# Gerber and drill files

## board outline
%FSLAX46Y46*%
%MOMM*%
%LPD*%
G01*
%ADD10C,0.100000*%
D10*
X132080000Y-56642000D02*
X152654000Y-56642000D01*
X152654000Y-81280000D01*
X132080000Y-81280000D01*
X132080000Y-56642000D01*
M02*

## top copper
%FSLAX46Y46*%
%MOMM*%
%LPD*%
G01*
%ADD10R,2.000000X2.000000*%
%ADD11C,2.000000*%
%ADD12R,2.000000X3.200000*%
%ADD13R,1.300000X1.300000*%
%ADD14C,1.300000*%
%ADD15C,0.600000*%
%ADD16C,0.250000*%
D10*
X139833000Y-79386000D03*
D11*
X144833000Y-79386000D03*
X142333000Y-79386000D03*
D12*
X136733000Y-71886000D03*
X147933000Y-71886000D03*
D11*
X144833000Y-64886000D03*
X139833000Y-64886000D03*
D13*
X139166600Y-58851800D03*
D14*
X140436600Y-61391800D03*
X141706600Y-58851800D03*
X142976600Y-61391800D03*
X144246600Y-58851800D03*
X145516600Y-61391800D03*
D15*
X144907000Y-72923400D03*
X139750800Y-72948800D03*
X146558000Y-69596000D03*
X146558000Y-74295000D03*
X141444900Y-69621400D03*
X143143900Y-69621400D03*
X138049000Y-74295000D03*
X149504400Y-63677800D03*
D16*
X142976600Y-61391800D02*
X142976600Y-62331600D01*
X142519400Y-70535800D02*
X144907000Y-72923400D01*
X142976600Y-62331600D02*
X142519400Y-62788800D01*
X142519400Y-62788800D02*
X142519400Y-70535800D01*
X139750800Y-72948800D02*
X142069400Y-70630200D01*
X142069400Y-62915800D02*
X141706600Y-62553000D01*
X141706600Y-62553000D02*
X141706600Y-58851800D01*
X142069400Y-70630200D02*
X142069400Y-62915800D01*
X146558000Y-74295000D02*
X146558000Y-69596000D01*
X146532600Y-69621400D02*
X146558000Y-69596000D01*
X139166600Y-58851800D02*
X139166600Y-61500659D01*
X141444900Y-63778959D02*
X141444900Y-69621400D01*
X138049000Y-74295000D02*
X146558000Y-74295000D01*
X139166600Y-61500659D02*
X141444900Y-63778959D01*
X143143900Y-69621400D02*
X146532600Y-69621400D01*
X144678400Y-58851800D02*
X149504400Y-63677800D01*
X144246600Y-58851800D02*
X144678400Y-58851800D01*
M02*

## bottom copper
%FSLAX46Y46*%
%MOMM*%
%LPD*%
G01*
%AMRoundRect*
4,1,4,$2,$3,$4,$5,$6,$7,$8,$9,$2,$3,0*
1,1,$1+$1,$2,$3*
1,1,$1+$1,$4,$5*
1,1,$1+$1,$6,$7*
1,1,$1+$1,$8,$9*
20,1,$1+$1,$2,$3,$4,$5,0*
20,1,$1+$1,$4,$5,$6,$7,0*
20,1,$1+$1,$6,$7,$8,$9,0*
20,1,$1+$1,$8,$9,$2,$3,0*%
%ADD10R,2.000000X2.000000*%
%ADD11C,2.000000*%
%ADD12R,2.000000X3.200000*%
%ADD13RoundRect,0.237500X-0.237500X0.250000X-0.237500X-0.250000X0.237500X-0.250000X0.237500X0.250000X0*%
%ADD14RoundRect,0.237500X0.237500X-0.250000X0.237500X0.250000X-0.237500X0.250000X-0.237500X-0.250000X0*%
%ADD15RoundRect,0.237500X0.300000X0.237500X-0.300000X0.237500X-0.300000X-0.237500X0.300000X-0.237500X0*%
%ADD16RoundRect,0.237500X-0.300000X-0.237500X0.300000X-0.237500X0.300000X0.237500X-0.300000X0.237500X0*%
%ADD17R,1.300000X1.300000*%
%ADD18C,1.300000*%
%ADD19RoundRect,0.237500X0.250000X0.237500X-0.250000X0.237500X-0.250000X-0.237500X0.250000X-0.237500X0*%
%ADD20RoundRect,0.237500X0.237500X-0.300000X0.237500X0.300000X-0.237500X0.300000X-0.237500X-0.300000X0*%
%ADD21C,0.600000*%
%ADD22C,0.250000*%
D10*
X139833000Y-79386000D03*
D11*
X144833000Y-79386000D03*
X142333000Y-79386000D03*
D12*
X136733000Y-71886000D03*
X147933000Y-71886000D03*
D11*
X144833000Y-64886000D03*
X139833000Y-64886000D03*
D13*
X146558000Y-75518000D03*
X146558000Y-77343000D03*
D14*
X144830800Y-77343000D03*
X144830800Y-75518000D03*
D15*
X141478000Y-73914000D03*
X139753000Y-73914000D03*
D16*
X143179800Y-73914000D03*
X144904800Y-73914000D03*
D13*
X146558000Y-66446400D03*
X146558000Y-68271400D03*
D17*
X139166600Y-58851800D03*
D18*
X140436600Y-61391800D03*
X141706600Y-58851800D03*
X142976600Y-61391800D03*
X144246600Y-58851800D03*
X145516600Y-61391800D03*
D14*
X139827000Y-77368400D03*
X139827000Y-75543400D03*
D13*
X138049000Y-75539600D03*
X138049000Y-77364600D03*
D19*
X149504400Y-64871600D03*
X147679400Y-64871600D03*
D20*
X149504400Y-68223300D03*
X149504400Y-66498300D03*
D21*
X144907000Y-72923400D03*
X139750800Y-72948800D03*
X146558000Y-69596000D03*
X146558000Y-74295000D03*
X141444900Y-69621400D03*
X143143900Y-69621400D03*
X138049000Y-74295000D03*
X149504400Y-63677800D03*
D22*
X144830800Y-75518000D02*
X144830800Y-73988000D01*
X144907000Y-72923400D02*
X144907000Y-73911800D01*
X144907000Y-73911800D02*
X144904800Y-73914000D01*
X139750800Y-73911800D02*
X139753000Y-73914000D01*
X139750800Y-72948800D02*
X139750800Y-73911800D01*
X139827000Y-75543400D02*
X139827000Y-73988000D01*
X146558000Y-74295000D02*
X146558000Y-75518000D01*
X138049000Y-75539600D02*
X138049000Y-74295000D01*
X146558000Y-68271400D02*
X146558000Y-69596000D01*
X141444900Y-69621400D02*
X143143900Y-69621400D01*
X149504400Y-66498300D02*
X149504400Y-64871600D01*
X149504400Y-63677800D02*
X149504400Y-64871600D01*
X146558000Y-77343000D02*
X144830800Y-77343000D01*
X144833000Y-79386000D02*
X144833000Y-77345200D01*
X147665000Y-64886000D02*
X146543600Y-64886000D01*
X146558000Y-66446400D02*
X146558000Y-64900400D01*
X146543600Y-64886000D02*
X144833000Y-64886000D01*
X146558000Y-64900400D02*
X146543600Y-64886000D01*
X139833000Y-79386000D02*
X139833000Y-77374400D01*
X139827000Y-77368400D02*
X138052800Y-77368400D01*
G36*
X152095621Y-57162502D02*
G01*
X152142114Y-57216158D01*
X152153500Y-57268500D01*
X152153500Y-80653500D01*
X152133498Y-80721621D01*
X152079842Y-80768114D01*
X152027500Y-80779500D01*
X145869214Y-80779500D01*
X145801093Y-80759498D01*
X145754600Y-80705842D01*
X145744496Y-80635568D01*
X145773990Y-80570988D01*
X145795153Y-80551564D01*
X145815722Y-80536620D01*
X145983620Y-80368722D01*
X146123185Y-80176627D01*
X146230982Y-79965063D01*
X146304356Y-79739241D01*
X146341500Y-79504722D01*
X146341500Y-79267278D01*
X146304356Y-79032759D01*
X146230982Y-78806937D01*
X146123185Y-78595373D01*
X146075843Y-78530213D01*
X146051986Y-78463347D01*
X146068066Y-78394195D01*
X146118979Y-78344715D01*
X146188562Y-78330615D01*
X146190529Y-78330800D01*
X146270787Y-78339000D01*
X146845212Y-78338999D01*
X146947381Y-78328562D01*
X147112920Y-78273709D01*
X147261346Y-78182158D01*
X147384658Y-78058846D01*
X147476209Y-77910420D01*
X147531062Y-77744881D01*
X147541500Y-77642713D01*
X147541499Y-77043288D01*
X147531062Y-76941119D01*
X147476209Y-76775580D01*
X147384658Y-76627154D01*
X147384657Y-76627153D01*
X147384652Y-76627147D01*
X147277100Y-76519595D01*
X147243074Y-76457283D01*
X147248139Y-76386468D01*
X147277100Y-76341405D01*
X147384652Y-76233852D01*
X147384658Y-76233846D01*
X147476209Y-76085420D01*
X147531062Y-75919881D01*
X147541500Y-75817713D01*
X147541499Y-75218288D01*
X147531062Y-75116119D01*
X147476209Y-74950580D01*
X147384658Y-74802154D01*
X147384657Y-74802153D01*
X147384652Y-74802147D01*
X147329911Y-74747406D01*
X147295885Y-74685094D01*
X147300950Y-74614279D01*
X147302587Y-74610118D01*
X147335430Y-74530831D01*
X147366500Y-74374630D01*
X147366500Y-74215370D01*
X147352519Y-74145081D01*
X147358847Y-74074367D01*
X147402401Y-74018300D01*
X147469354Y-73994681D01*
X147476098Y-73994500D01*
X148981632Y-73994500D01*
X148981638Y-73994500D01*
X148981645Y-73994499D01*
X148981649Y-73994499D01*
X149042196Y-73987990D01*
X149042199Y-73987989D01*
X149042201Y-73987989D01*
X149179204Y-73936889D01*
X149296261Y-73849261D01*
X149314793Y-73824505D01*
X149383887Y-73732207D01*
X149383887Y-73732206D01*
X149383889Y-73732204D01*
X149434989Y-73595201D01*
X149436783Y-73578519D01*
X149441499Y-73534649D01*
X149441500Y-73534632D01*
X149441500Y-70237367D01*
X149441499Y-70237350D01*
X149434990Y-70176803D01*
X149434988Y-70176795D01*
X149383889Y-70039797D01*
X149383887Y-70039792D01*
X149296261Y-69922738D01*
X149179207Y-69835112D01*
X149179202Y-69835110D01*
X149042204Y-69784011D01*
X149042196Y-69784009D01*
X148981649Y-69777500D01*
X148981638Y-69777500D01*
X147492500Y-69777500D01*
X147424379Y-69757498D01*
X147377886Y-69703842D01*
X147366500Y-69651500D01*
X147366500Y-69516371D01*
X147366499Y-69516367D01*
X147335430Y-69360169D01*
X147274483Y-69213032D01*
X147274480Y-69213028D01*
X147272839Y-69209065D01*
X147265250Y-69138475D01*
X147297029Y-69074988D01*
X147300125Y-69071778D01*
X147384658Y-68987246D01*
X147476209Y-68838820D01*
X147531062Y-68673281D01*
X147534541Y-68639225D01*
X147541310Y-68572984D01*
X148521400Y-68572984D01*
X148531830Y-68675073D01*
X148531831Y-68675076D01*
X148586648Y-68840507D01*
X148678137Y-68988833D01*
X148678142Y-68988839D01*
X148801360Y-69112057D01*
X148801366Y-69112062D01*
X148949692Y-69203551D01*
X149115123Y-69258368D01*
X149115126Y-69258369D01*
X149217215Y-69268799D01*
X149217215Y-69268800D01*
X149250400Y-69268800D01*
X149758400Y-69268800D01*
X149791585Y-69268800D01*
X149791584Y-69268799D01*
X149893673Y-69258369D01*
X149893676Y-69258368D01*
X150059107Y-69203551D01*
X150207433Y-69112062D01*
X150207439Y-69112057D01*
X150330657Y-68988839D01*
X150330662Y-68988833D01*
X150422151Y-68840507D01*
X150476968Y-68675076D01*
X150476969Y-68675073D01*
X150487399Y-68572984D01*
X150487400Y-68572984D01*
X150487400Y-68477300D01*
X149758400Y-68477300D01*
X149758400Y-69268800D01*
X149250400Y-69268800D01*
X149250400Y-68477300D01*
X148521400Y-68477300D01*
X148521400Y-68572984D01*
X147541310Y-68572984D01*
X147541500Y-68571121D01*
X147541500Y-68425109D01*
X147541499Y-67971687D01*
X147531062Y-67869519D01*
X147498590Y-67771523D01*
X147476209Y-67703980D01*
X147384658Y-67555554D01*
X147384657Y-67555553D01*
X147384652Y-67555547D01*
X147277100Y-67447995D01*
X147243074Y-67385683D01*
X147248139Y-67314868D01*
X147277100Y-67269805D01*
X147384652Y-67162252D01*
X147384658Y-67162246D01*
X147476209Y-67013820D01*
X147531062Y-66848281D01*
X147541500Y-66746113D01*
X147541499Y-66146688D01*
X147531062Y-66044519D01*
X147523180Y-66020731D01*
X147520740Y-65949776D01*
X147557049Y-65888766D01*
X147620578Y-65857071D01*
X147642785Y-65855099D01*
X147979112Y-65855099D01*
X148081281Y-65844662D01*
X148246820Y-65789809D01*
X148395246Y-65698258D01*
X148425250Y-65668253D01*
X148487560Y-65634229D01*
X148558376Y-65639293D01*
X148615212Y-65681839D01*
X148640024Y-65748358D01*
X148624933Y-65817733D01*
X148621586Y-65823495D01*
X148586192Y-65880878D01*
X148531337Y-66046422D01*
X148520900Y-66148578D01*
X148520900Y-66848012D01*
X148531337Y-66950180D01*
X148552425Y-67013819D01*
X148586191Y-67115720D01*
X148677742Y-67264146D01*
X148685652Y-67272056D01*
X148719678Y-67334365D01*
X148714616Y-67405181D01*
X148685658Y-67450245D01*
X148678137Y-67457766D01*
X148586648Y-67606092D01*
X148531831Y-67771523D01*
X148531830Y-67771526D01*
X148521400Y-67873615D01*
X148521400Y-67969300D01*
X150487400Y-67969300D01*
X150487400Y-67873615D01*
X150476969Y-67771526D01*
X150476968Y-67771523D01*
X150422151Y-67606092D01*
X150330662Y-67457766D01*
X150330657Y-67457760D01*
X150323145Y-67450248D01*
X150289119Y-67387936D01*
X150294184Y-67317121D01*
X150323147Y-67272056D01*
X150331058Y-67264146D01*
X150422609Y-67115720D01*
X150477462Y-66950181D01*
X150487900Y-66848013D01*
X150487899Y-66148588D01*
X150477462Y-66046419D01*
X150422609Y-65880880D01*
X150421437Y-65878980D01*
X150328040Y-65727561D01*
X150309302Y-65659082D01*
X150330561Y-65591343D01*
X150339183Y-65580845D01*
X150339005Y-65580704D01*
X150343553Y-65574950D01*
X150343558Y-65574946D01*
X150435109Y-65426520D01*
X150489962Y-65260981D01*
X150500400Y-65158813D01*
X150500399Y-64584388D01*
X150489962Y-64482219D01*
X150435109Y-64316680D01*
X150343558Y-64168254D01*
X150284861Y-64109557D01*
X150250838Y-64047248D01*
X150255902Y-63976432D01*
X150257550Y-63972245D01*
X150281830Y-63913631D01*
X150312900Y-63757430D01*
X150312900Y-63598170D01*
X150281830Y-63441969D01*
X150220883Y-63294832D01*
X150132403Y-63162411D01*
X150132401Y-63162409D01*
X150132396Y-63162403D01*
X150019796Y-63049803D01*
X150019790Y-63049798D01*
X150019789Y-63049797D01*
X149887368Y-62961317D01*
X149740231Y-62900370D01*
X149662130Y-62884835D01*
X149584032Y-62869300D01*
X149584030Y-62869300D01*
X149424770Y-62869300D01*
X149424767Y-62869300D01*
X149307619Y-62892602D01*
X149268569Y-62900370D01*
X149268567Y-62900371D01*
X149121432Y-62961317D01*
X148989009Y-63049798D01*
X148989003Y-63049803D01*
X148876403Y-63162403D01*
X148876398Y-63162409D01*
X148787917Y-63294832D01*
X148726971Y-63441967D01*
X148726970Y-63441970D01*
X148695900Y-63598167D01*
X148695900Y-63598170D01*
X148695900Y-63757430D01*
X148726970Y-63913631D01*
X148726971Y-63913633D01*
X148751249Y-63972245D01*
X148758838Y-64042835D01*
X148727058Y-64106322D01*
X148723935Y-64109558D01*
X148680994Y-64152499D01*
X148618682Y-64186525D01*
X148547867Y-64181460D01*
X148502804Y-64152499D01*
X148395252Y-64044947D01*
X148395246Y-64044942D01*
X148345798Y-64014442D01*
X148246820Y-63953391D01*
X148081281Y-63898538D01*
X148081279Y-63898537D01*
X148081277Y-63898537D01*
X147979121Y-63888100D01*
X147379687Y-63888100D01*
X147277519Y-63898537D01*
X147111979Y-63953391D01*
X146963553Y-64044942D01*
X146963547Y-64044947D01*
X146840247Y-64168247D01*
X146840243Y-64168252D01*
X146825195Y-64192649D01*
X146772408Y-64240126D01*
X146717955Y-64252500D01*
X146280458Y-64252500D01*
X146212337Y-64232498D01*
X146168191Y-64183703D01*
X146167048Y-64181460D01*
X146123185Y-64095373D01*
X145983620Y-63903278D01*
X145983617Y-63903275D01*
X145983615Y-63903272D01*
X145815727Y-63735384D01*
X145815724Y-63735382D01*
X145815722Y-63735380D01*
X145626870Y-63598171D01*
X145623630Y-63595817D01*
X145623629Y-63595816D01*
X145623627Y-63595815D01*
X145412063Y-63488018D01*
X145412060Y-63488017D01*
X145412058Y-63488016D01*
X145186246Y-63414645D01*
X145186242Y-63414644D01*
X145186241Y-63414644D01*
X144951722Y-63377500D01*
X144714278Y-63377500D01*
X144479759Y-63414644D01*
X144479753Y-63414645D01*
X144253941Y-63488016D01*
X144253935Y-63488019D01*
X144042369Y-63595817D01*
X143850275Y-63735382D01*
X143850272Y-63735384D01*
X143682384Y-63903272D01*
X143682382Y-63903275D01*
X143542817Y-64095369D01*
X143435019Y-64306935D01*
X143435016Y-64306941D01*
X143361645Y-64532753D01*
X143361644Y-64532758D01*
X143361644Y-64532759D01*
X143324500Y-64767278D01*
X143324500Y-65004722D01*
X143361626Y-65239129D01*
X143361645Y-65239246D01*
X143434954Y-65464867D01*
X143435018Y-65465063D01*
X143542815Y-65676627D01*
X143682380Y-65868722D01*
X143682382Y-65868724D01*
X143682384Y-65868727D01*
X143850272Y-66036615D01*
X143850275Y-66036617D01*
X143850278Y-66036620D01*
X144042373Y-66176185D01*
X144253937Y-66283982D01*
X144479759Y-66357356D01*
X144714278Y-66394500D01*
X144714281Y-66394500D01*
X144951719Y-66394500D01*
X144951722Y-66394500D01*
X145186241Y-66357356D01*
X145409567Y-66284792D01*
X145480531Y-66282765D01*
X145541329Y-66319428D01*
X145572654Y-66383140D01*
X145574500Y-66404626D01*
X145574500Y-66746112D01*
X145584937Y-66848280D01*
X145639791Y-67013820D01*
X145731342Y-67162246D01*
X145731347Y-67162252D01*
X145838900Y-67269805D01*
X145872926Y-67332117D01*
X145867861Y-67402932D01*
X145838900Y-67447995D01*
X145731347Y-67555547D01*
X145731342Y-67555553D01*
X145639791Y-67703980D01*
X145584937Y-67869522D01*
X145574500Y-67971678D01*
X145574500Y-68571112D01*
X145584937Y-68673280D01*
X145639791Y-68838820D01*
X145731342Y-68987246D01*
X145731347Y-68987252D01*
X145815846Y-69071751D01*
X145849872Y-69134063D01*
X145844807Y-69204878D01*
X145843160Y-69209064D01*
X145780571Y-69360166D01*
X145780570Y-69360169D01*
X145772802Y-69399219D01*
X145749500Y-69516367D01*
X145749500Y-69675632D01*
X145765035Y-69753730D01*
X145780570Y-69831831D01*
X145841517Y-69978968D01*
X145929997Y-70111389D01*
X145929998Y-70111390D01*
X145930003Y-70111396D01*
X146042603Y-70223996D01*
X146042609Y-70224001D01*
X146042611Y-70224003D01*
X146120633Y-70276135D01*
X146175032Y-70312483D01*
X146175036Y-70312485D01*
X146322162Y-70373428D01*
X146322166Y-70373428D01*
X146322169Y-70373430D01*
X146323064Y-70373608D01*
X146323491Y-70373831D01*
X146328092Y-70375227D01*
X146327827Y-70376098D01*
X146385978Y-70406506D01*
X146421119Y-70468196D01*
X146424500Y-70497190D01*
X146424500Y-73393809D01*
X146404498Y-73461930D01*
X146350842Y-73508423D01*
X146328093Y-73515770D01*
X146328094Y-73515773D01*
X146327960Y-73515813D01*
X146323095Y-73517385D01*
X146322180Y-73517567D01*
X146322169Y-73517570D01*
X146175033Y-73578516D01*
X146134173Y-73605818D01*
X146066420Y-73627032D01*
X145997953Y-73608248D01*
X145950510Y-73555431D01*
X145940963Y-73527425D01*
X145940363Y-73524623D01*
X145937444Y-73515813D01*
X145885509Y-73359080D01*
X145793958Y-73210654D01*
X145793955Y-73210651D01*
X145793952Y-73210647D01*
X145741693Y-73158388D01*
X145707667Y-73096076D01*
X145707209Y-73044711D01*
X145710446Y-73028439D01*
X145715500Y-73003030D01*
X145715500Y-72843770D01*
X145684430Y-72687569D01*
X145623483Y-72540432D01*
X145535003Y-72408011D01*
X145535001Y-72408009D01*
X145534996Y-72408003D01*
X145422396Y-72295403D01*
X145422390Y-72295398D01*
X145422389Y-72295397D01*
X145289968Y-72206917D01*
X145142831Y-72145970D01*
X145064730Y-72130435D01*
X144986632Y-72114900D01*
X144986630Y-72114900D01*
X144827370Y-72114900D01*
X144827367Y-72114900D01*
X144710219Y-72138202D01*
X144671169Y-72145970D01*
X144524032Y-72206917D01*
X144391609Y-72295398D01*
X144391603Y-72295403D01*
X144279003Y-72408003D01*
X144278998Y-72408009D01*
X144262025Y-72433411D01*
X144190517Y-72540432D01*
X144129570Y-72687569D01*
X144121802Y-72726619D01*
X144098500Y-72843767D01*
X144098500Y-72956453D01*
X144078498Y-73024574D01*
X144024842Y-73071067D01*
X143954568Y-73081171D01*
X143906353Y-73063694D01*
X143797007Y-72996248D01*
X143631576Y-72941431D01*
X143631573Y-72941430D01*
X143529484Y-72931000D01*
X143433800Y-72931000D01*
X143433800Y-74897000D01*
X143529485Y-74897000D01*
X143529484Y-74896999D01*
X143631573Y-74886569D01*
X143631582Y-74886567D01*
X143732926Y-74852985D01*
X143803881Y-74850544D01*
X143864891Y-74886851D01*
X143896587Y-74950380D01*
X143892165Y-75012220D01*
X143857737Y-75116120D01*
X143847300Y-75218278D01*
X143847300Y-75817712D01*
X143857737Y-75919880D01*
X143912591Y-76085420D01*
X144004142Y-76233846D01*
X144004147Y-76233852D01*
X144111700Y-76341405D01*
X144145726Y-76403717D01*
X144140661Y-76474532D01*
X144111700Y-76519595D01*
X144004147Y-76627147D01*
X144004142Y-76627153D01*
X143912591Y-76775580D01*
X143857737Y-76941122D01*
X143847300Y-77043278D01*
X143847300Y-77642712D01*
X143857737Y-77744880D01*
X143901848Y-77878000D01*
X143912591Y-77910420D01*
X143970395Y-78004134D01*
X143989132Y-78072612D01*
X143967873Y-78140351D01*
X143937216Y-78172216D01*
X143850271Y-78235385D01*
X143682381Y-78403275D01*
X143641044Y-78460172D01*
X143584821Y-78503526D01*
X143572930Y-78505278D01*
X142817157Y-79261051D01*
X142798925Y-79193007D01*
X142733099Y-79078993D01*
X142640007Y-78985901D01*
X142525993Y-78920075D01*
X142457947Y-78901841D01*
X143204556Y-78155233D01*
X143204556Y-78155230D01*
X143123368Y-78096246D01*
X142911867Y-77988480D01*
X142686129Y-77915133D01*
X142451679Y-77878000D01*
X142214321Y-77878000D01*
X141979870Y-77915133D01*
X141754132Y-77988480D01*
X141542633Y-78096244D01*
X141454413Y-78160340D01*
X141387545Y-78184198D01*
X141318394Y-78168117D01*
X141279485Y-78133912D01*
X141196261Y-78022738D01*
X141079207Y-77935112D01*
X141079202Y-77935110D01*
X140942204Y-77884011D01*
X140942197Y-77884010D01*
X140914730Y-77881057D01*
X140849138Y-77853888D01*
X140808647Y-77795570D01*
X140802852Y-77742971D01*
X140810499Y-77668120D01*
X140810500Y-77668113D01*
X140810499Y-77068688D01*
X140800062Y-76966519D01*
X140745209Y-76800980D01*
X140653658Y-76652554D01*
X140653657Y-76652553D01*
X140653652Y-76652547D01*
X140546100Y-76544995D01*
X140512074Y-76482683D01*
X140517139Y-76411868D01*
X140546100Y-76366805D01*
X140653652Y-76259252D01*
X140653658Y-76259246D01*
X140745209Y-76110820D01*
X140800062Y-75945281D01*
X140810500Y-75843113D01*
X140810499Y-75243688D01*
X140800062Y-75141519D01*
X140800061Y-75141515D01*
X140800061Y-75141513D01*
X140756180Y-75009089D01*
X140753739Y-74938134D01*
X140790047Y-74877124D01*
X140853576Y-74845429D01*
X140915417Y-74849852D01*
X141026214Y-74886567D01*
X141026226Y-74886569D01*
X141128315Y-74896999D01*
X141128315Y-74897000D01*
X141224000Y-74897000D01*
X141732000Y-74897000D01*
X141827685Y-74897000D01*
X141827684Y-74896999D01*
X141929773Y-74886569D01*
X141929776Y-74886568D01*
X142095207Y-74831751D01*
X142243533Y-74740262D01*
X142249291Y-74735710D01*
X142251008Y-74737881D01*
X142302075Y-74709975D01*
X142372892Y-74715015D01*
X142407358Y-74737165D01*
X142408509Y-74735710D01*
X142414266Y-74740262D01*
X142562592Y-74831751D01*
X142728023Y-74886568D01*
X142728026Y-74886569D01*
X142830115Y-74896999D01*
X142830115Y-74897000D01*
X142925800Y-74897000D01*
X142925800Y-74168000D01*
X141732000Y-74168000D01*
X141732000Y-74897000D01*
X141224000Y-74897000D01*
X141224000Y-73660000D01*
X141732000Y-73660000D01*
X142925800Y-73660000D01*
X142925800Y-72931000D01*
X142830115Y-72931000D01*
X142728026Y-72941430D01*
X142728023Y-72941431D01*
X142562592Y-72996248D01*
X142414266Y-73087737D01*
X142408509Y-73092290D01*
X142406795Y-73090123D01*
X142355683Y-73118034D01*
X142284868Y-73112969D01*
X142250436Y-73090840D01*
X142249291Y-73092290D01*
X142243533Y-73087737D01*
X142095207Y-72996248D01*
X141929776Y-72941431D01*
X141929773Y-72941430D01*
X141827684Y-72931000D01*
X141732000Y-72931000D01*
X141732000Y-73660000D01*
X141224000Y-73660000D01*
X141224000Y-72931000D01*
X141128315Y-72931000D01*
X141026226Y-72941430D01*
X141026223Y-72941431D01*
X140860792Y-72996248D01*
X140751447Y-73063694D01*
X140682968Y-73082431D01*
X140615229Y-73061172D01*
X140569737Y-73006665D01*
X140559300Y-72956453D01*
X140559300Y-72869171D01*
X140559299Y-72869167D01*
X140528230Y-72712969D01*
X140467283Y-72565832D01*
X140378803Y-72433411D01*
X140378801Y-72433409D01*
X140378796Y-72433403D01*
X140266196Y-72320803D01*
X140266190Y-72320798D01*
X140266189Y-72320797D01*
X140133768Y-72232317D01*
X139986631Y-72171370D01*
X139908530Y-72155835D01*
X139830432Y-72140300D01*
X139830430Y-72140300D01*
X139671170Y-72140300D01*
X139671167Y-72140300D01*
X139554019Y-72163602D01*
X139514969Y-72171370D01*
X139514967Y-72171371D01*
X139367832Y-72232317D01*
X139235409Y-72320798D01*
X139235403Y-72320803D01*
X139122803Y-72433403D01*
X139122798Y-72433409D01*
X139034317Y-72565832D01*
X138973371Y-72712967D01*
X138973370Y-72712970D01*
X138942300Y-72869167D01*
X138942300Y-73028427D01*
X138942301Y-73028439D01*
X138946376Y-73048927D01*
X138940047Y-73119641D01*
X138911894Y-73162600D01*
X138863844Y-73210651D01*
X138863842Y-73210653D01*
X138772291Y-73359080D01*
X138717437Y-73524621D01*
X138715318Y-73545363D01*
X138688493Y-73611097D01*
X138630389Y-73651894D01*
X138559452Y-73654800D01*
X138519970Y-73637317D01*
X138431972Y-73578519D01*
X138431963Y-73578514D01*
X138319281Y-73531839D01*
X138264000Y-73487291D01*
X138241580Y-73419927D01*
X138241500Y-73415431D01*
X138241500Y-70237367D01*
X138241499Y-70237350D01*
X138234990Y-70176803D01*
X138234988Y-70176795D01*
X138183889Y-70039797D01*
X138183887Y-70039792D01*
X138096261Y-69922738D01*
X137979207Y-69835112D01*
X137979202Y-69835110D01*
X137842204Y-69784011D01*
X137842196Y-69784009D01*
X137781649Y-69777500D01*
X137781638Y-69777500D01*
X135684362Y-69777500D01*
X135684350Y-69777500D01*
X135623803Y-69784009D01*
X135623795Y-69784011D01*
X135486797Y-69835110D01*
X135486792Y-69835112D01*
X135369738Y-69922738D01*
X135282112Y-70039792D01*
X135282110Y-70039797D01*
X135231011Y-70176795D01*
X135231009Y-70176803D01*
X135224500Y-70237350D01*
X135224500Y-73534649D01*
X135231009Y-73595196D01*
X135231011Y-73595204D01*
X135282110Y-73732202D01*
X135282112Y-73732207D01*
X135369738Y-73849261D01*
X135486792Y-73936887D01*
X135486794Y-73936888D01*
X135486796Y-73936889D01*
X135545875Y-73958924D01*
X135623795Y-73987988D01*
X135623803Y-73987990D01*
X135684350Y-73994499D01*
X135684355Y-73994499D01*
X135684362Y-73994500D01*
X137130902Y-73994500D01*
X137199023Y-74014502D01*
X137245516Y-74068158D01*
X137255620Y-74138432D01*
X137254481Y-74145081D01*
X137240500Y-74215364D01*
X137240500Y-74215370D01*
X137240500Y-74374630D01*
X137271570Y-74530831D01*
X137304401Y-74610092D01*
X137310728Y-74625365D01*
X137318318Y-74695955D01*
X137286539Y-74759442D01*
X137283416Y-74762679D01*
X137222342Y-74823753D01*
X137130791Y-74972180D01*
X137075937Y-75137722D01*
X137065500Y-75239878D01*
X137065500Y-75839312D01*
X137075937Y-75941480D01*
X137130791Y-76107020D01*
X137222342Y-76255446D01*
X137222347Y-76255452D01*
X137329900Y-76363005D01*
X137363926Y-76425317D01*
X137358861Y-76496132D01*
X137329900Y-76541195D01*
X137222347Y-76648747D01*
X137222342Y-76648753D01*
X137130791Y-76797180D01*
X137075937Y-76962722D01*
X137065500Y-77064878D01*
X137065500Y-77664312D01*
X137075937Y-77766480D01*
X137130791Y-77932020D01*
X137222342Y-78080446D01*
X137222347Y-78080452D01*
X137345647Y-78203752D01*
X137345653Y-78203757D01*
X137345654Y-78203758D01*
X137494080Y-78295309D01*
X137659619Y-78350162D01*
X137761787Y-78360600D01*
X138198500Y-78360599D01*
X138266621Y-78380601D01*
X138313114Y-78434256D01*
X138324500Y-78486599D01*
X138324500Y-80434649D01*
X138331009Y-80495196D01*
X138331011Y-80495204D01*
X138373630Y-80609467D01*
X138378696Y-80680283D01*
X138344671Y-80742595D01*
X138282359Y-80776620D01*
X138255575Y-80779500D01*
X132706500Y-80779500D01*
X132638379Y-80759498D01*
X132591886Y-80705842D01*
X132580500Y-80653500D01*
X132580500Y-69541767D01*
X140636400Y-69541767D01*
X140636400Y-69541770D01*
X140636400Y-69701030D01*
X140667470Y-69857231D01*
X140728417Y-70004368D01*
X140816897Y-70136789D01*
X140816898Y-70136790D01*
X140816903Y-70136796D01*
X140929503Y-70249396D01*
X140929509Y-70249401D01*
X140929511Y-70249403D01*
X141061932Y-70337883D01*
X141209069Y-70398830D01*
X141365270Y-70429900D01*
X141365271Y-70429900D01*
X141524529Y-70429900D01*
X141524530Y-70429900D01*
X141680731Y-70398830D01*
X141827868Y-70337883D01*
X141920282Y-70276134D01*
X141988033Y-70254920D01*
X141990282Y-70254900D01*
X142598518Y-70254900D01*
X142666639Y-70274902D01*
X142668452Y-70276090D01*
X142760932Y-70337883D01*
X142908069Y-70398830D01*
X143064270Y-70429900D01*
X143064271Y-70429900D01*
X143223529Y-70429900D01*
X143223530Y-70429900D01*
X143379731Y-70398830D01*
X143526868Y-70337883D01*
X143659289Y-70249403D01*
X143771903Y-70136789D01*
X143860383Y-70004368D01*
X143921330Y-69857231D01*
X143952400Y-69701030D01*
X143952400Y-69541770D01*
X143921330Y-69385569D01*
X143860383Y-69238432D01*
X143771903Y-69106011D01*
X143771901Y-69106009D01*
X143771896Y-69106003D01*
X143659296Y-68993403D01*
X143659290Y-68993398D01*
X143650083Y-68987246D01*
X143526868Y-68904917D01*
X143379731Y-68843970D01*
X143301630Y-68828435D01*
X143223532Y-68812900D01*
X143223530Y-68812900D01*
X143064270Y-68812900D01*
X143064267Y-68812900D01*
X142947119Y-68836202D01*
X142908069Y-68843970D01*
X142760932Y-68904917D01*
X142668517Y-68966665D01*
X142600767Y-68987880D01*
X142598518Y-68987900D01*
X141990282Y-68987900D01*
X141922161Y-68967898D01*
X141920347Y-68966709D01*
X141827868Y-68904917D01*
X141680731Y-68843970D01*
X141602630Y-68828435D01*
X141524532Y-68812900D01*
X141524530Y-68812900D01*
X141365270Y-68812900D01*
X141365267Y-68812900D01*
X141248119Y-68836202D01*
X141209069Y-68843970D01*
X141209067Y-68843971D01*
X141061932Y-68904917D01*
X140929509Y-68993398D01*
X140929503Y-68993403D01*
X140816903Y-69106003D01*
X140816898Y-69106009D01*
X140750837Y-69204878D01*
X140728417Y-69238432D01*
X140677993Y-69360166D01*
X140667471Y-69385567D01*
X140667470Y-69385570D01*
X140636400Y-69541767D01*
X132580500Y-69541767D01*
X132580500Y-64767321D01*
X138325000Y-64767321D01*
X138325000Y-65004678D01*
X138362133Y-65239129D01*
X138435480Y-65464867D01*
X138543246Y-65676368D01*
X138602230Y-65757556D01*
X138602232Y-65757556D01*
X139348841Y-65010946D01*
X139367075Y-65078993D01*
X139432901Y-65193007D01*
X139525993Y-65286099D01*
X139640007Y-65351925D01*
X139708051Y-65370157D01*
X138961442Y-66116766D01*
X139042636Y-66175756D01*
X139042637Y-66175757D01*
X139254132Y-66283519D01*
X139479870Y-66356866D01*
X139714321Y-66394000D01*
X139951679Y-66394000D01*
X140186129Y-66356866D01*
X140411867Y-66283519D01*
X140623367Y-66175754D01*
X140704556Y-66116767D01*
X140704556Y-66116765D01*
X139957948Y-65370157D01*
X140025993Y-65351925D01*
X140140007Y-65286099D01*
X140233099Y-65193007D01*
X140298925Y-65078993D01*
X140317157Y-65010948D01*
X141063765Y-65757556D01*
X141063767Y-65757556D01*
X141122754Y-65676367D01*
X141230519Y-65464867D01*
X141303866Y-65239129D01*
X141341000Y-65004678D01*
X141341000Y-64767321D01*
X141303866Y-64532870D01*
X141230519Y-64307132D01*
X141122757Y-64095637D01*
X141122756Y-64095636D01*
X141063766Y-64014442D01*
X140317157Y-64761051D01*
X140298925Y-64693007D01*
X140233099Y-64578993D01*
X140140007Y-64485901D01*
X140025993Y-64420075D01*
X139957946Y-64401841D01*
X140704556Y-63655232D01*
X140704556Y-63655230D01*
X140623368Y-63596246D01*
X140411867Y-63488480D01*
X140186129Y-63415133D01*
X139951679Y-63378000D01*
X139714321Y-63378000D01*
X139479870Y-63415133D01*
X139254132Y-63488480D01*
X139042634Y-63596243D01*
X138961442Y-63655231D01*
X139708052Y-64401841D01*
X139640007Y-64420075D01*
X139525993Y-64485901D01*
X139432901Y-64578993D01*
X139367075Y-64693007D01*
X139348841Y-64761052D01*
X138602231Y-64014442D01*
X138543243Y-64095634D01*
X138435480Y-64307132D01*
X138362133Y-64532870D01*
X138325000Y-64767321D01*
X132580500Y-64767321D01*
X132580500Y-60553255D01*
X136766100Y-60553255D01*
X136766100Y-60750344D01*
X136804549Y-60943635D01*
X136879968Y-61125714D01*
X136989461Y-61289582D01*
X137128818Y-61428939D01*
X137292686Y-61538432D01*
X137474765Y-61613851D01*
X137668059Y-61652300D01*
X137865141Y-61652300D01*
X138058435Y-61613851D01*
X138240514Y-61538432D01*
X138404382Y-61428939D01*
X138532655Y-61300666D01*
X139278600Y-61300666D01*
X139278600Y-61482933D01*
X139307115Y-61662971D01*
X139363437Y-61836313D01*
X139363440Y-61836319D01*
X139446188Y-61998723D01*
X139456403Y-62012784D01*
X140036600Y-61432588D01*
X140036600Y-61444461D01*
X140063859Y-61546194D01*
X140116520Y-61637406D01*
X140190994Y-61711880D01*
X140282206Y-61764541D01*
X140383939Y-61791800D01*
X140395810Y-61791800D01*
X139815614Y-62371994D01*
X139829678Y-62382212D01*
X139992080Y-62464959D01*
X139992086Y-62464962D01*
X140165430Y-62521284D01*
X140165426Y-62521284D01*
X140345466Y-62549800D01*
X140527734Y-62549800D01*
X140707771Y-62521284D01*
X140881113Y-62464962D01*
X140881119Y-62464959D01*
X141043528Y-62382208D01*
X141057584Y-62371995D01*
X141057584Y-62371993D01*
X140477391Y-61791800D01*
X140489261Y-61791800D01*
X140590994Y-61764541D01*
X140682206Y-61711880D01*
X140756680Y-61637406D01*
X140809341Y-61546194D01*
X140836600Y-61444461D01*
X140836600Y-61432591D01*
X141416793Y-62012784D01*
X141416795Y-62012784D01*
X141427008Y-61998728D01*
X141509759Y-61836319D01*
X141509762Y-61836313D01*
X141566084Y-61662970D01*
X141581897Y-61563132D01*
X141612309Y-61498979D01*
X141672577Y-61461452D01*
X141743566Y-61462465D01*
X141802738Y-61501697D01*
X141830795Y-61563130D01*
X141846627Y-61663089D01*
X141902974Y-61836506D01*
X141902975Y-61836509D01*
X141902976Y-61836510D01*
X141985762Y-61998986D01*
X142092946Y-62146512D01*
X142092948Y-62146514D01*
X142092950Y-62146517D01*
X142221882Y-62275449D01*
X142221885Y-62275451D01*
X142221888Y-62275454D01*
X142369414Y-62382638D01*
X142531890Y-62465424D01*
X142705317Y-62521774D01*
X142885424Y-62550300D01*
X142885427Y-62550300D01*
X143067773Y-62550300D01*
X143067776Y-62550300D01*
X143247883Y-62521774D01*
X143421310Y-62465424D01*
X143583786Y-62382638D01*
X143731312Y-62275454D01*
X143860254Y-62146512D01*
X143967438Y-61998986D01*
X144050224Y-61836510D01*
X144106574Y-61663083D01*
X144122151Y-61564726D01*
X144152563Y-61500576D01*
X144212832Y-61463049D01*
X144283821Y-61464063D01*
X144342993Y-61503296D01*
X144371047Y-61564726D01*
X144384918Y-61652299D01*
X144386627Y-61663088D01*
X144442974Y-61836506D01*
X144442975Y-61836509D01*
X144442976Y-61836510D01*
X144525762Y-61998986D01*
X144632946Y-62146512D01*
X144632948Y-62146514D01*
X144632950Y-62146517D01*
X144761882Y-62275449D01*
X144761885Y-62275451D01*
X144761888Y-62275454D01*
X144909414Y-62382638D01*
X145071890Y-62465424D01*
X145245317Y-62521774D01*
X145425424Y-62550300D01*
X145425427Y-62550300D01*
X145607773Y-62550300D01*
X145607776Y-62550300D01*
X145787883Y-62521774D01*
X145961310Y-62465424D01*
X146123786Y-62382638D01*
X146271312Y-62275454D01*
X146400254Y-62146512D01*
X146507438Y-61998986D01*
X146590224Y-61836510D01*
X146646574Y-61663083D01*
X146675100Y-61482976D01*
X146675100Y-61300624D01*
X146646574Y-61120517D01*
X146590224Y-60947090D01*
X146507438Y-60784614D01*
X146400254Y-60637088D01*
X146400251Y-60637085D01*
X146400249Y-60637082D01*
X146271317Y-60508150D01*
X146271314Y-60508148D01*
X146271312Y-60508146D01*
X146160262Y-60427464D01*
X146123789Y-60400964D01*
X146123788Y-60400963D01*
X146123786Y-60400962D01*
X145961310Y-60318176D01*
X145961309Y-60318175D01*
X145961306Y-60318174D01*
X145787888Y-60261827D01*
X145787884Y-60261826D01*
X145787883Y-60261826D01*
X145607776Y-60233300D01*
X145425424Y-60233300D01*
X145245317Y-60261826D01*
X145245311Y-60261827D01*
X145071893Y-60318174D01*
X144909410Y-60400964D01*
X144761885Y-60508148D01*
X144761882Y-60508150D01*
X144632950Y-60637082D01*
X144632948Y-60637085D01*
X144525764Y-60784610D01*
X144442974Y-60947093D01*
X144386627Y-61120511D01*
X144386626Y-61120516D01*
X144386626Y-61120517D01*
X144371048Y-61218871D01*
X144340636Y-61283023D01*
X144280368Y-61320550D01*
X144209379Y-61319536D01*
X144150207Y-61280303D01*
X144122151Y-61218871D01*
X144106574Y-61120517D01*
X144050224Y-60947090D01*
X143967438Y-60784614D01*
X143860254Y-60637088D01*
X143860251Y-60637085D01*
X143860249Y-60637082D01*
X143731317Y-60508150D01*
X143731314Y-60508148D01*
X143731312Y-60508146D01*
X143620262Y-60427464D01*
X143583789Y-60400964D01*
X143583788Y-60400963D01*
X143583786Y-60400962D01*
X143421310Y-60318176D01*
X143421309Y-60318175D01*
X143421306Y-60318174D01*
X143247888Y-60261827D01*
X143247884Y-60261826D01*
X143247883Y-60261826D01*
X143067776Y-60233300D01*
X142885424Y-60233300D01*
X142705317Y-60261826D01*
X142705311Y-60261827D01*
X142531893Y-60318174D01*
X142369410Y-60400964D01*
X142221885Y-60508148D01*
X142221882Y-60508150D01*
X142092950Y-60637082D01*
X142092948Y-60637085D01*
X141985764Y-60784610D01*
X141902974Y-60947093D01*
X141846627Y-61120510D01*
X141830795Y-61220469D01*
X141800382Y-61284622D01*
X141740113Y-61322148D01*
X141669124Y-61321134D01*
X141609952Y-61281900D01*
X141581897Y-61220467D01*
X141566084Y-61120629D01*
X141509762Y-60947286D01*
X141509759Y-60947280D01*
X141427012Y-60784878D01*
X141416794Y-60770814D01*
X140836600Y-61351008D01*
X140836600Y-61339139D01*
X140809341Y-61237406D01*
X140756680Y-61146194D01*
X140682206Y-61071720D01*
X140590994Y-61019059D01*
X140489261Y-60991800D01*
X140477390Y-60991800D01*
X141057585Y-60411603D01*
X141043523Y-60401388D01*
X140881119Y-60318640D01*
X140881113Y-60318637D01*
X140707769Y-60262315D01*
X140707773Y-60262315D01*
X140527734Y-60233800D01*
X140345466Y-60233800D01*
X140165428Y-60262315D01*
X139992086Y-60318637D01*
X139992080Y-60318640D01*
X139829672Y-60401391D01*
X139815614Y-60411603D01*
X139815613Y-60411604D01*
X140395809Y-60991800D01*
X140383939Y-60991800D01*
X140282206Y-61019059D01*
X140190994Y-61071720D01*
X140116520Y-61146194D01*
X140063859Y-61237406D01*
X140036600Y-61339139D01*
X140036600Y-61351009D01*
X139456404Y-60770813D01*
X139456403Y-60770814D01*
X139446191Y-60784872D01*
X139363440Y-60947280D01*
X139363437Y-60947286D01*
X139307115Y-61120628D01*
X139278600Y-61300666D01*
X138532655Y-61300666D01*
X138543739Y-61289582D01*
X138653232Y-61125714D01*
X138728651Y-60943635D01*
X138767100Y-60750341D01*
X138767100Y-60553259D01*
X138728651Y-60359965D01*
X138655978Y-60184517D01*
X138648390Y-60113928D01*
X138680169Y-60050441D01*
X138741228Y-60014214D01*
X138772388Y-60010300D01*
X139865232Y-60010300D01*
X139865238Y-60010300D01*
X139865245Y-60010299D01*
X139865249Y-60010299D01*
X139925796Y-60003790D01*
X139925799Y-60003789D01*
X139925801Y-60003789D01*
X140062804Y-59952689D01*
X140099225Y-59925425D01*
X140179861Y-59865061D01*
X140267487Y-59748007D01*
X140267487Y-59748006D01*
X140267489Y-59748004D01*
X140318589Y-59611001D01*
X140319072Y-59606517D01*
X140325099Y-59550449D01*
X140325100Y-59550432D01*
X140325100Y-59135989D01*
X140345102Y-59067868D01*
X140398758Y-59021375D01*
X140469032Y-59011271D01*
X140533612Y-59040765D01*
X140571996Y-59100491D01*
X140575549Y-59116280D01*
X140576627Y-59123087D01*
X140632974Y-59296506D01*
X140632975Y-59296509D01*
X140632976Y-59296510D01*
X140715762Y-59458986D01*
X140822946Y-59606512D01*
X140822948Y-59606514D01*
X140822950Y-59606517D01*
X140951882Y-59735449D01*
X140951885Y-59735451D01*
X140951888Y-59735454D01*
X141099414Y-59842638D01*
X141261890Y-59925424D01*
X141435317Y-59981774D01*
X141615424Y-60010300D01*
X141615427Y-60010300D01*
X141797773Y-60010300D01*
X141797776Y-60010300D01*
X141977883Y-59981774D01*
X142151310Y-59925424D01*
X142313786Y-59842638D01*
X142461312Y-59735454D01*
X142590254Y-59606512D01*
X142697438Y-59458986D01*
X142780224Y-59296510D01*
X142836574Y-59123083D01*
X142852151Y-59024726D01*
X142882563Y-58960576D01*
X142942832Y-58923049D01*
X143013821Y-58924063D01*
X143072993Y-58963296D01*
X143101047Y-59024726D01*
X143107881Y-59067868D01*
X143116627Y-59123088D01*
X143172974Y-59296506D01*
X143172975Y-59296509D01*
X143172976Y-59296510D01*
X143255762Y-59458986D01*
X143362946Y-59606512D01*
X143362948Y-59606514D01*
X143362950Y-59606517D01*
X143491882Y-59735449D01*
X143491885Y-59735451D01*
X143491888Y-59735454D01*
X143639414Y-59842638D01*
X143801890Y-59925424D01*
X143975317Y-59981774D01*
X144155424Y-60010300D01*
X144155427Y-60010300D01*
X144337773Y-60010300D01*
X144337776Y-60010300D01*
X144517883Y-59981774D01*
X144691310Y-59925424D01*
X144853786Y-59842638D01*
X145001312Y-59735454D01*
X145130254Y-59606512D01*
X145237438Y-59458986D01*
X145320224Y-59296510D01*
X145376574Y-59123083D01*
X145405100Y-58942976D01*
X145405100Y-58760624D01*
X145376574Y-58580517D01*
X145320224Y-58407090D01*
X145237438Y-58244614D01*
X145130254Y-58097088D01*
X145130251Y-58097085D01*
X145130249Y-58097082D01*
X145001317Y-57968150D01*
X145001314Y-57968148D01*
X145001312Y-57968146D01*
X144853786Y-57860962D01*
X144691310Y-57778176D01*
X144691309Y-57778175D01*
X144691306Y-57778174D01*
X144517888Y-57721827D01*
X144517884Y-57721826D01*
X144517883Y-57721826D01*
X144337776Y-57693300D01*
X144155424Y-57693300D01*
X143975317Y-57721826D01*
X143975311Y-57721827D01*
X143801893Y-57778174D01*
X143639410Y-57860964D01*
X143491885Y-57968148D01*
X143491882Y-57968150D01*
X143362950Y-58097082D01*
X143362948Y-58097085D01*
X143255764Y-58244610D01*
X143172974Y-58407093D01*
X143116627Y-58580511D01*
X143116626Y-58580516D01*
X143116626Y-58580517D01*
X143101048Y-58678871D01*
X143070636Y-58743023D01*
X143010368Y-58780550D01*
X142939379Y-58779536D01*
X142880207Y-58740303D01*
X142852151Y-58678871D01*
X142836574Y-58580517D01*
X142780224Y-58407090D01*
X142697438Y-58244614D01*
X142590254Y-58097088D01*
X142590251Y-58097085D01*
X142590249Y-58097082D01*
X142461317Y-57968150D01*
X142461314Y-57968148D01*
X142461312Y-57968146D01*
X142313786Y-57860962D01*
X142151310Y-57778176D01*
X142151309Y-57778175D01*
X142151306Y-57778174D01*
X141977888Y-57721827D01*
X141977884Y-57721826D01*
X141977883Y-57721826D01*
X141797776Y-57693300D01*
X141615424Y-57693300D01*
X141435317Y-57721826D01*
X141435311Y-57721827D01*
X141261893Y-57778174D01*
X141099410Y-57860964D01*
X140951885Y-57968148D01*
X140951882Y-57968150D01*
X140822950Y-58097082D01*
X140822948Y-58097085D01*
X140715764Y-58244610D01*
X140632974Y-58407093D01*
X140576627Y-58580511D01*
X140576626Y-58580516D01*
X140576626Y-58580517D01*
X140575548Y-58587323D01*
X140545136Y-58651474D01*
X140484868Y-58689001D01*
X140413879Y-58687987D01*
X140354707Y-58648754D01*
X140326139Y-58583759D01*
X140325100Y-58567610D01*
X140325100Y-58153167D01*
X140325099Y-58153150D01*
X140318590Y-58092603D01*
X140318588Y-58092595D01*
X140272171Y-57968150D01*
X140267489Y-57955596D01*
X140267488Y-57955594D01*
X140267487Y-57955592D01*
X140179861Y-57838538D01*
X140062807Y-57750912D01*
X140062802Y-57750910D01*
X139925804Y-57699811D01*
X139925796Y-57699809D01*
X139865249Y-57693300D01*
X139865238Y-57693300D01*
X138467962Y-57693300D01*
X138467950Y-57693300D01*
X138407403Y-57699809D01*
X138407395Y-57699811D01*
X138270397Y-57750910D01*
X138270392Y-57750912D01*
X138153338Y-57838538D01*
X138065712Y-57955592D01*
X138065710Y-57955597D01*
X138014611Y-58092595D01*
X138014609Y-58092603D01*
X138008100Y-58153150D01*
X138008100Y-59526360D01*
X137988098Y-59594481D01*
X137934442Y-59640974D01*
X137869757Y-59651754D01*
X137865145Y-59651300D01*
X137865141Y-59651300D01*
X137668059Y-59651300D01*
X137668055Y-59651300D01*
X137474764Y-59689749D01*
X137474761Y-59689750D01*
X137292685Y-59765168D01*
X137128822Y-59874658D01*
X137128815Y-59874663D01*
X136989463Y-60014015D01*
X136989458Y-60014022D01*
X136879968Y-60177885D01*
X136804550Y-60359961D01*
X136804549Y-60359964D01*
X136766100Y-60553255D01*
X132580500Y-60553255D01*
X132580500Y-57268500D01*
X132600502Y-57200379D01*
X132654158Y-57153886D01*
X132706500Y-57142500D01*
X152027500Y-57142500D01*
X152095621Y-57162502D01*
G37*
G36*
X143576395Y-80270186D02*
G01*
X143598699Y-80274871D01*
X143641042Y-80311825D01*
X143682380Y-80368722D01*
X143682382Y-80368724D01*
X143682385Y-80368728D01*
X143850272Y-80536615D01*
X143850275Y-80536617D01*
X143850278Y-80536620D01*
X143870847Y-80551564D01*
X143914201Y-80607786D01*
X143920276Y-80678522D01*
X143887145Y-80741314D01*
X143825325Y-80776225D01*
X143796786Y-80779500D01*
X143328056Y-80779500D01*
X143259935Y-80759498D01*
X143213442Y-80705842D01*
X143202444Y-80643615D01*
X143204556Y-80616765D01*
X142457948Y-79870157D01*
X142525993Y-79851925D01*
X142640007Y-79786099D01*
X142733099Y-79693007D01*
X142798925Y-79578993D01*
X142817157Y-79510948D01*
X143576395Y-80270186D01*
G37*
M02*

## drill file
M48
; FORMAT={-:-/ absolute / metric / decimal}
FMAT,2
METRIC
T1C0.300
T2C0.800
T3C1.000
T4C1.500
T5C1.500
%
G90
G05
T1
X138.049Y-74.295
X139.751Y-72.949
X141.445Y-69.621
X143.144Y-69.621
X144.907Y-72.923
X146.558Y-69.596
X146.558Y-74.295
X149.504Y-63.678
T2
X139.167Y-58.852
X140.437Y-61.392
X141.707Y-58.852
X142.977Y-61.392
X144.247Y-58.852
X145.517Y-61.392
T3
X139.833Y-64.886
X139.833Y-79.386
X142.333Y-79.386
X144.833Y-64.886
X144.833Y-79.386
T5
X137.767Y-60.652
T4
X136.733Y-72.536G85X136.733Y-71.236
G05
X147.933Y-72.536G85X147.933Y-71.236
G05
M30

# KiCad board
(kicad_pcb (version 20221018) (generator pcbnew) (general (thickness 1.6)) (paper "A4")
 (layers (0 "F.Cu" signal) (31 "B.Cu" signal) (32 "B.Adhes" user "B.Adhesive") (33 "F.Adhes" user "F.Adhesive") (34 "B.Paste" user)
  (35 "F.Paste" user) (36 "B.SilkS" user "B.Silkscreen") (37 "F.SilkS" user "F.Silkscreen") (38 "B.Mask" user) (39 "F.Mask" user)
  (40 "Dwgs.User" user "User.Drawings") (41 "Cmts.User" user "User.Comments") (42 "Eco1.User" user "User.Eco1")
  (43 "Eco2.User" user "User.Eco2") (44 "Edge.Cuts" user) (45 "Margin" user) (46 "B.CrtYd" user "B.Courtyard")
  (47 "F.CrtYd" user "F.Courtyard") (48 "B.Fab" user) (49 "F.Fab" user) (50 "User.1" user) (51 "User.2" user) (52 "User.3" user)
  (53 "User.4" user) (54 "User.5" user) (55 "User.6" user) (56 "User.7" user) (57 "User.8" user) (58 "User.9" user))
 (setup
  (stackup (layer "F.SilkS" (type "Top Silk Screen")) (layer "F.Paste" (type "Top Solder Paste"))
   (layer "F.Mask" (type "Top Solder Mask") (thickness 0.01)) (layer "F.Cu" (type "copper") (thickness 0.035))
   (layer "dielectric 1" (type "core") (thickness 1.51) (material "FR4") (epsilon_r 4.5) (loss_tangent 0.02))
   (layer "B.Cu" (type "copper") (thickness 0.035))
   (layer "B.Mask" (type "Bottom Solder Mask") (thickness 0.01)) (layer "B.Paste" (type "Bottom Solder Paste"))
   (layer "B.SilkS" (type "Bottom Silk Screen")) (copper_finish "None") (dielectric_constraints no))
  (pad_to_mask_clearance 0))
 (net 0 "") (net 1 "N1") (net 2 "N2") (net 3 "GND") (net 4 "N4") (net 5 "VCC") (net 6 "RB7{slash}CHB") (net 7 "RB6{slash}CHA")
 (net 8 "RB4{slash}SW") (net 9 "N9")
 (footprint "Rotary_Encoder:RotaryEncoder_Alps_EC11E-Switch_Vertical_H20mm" (layer "F.Cu") (at 139.833 79.386 90)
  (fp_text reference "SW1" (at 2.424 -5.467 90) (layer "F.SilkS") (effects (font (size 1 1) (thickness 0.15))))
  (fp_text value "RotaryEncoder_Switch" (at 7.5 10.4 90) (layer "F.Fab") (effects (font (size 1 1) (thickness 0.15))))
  (pad "A" thru_hole rect (at 0 0 90) (size 2 2) (drill 1) (layers "*.Cu" "*.Mask") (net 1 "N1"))
  (pad "B" thru_hole circle (at 0 5 90) (size 2 2) (drill 1) (layers "*.Cu" "*.Mask") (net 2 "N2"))
  (pad "C" thru_hole circle (at 0 2.5 90) (size 2 2) (drill 1) (layers "*.Cu" "*.Mask") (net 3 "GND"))
  (pad "MP" thru_hole rect (at 7.5 -3.1 90) (size 3.2 2) (drill oval 2.8 1.5) (layers "*.Cu" "*.Mask"))
  (pad "MP" thru_hole rect (at 7.5 8.1 90) (size 3.2 2) (drill oval 2.8 1.5) (layers "*.Cu" "*.Mask"))
  (pad "S1" thru_hole circle (at 14.5 5 90) (size 2 2) (drill 1) (layers "*.Cu" "*.Mask") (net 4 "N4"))
  (pad "S2" thru_hole circle (at 14.5 0 90) (size 2 2) (drill 1) (layers "*.Cu" "*.Mask") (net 3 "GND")))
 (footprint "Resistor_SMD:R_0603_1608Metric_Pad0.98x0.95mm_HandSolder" (layer "B.Cu") (at 146.558 76.4305 -90)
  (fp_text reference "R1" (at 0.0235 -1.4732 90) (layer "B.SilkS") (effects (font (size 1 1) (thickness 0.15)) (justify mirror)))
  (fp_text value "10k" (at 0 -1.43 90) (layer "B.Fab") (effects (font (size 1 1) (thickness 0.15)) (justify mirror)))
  (pad "1" smd roundrect (at -0.9125 0 270) (size 0.975 0.95) (layers "B.Cu" "B.Paste" "B.Mask") (roundrect_rratio 0.25) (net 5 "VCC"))
  (pad "2" smd roundrect (at 0.9125 0 270) (size 0.975 0.95) (layers "B.Cu" "B.Paste" "B.Mask") (roundrect_rratio 0.25) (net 2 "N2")))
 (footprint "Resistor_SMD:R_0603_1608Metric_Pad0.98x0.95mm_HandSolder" (layer "B.Cu") (at 144.8308 76.4305 90)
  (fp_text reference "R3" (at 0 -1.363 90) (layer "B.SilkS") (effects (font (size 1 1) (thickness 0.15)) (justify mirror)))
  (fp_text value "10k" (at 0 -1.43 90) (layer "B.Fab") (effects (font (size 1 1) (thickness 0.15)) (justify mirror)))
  (pad "1" smd roundrect (at -0.9125 0 90) (size 0.975 0.95) (layers "B.Cu" "B.Paste" "B.Mask") (roundrect_rratio 0.25) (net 2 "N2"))
  (pad "2" smd roundrect (at 0.9125 0 90) (size 0.975 0.95) (layers "B.Cu" "B.Paste" "B.Mask") (roundrect_rratio 0.25)
   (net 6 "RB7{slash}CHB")))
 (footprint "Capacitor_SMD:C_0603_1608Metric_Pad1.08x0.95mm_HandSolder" (layer "B.Cu") (at 140.6155 73.914 180)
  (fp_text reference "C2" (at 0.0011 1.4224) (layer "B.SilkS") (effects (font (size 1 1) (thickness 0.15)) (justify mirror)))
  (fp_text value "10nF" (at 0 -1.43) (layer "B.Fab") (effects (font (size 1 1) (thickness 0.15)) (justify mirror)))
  (pad "1" smd roundrect (at -0.8625 0 180) (size 1.075 0.95) (layers "B.Cu" "B.Paste" "B.Mask") (roundrect_rratio 0.25) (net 3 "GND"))
  (pad "2" smd roundrect (at 0.8625 0 180) (size 1.075 0.95) (layers "B.Cu" "B.Paste" "B.Mask") (roundrect_rratio 0.25)
   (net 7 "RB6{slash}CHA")))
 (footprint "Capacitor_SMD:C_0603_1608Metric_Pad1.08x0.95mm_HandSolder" (layer "B.Cu") (at 144.0423 73.914)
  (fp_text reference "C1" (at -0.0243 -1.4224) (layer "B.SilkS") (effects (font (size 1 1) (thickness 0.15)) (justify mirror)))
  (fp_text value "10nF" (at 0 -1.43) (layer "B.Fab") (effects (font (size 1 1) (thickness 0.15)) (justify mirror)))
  (pad "1" smd roundrect (at -0.8625 0) (size 1.075 0.95) (layers "B.Cu" "B.Paste" "B.Mask") (roundrect_rratio 0.25) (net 3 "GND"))
  (pad "2" smd roundrect (at 0.8625 0) (size 1.075 0.95) (layers "B.Cu" "B.Paste" "B.Mask") (roundrect_rratio 0.25) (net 6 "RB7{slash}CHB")))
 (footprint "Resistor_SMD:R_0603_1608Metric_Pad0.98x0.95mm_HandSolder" (layer "B.Cu") (at 146.558 67.3589 -90)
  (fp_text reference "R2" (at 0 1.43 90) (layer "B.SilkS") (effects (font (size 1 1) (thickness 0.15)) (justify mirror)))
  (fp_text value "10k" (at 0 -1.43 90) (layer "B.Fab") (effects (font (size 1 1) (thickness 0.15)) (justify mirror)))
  (pad "1" smd roundrect (at -0.9125 0 270) (size 0.975 0.95) (layers "B.Cu" "B.Paste" "B.Mask") (roundrect_rratio 0.25) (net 4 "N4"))
  (pad "2" smd roundrect (at 0.9125 0 270) (size 0.975 0.95) (layers "B.Cu" "B.Paste" "B.Mask") (roundrect_rratio 0.25) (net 5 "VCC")))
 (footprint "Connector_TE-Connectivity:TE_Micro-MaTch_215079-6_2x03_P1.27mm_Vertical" (layer "B.Cu") (at 139.1666 58.8518 -90)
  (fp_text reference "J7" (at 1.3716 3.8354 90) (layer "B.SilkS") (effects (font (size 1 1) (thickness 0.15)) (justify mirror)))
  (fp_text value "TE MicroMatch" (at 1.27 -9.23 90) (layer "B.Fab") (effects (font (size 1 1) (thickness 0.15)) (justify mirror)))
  (pad "" np_thru_hole circle (at 1.8 1.4 270) (size 1.5 1.5) (drill 1.5) (layers "*.Cu" "*.Mask"))
  (pad "1" thru_hole rect (at 0 0 270) (size 1.3 1.3) (drill 0.8) (layers "*.Cu" "*.Mask") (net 5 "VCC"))
  (pad "2" thru_hole circle (at 2.54 -1.27 270) (size 1.3 1.3) (drill 0.8) (layers "*.Cu" "*.Mask") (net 3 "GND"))
  (pad "3" thru_hole circle (at 0 -2.54 270) (size 1.3 1.3) (drill 0.8) (layers "*.Cu" "*.Mask") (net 7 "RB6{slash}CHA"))
  (pad "4" thru_hole circle (at 2.54 -3.81 270) (size 1.3 1.3) (drill 0.8) (layers "*.Cu" "*.Mask") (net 6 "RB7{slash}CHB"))
  (pad "5" thru_hole circle (at 0 -5.08 270) (size 1.3 1.3) (drill 0.8) (layers "*.Cu" "*.Mask") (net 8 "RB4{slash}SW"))
  (pad "6" thru_hole circle (at 2.54 -6.35 270) (size 1.3 1.3) (drill 0.8) (layers "*.Cu" "*.Mask") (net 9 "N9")))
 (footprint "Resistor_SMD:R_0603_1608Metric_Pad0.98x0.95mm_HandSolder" (layer "B.Cu") (at 139.827 76.4559 90)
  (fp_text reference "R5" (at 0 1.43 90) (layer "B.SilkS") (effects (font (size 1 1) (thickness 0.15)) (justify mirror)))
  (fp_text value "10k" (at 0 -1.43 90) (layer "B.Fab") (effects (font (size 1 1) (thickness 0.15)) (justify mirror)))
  (pad "1" smd roundrect (at -0.9125 0 90) (size 0.975 0.95) (layers "B.Cu" "B.Paste" "B.Mask") (roundrect_rratio 0.25) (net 1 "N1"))
  (pad "2" smd roundrect (at 0.9125 0 90) (size 0.975 0.95) (layers "B.Cu" "B.Paste" "B.Mask") (roundrect_rratio 0.25)
   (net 7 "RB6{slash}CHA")))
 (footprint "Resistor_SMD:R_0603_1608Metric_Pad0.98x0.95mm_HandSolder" (layer "B.Cu") (at 138.049 76.4521 -90)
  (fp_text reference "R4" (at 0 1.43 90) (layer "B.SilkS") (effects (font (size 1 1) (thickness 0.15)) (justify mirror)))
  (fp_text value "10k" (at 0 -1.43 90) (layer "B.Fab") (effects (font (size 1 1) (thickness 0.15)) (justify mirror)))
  (pad "1" smd roundrect (at -0.9125 0 270) (size 0.975 0.95) (layers "B.Cu" "B.Paste" "B.Mask") (roundrect_rratio 0.25) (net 5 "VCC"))
  (pad "2" smd roundrect (at 0.9125 0 270) (size 0.975 0.95) (layers "B.Cu" "B.Paste" "B.Mask") (roundrect_rratio 0.25) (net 1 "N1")))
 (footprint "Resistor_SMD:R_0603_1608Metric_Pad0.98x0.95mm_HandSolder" (layer "B.Cu") (at 148.5919 64.8716 180)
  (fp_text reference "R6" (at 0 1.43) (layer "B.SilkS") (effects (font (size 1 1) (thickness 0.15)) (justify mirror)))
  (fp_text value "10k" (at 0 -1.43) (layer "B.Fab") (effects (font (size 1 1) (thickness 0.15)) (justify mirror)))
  (pad "1" smd roundrect (at -0.9125 0 180) (size 0.975 0.95) (layers "B.Cu" "B.Paste" "B.Mask") (roundrect_rratio 0.25)
   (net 8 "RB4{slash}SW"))
  (pad "2" smd roundrect (at 0.9125 0 180) (size 0.975 0.95) (layers "B.Cu" "B.Paste" "B.Mask") (roundrect_rratio 0.25) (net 4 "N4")))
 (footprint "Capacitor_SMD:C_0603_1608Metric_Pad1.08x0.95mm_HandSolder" (layer "B.Cu") (at 149.5044 67.3608 90)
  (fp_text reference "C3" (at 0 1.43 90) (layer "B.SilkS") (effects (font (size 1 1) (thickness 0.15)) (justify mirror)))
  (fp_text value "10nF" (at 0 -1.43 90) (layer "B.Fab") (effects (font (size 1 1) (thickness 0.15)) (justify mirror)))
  (pad "1" smd roundrect (at -0.8625 0 90) (size 1.075 0.95) (layers "B.Cu" "B.Paste" "B.Mask") (roundrect_rratio 0.25) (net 3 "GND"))
  (pad "2" smd roundrect (at 0.8625 0 90) (size 1.075 0.95) (layers "B.Cu" "B.Paste" "B.Mask") (roundrect_rratio 0.25)
   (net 8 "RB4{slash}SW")))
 (gr_rect (start 132.08 56.642) (end 152.654 81.28) (stroke (width 0.1) (type solid)) (fill none) (layer "Edge.Cuts"))
 (segment (start 142.9766 61.3918) (end 142.9766 62.3316) (width 0.25) (layer "F.Cu") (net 6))
 (segment (start 142.5194 70.5358) (end 144.907 72.9234) (width 0.25) (layer "F.Cu") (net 6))
 (segment (start 142.9766 62.3316) (end 142.5194 62.7888) (width 0.25) (layer "F.Cu") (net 6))
 (segment (start 142.5194 62.7888) (end 142.5194 70.5358) (width 0.25) (layer "F.Cu") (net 6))
 (via (at 144.907 72.9234) (size 0.6) (drill 0.3) (layers "F.Cu" "B.Cu") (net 6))
 (segment (start 144.8308 75.518) (end 144.8308 73.988) (width 0.25) (layer "B.Cu") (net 6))
 (segment (start 144.907 72.9234) (end 144.907 73.9118) (width 0.25) (layer "B.Cu") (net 6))
 (segment (start 144.907 73.9118) (end 144.9048 73.914) (width 0.25) (layer "B.Cu") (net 6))
 (segment (start 139.7508 72.9488) (end 142.0694 70.6302) (width 0.25) (layer "F.Cu") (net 7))
 (segment (start 142.0694 62.9158) (end 141.7066 62.553) (width 0.25) (layer "F.Cu") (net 7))
 (segment (start 141.7066 62.553) (end 141.7066 58.8518) (width 0.25) (layer "F.Cu") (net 7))
 (segment (start 142.0694 70.6302) (end 142.0694 62.9158) (width 0.25) (layer "F.Cu") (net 7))
 (via (at 139.7508 72.9488) (size 0.6) (drill 0.3) (layers "F.Cu" "B.Cu") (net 7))
 (segment (start 139.7508 73.9118) (end 139.753 73.914) (width 0.25) (layer "B.Cu") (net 7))
 (segment (start 139.7508 72.9488) (end 139.7508 73.9118) (width 0.25) (layer "B.Cu") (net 7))
 (segment (start 139.827 75.5434) (end 139.827 73.988) (width 0.25) (layer "B.Cu") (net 7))
 (segment (start 146.558 74.295) (end 146.558 69.596) (width 0.25) (layer "F.Cu") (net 5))
 (segment (start 146.5326 69.6214) (end 146.558 69.596) (width 0.25) (layer "F.Cu") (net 5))
 (segment (start 139.1666 58.8518) (end 139.1666 61.500659) (width 0.25) (layer "F.Cu") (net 5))
 (segment (start 141.4449 63.778959) (end 141.4449 69.6214) (width 0.25) (layer "F.Cu") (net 5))
 (segment (start 138.049 74.295) (end 146.558 74.295) (width 0.25) (layer "F.Cu") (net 5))
 (segment (start 139.1666 61.500659) (end 141.4449 63.778959) (width 0.25) (layer "F.Cu") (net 5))
 (segment (start 143.1439 69.6214) (end 146.5326 69.6214) (width 0.25) (layer "F.Cu") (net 5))
 (via (at 146.558 69.596) (size 0.6) (drill 0.3) (layers "F.Cu" "B.Cu") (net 5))
 (via (at 146.558 74.295) (size 0.6) (drill 0.3) (layers "F.Cu" "B.Cu") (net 5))
 (via (at 141.4449 69.6214) (size 0.6) (drill 0.3) (layers "F.Cu" "B.Cu") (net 5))
 (via (at 143.1439 69.6214) (size 0.6) (drill 0.3) (layers "F.Cu" "B.Cu") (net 5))
 (via (at 138.049 74.295) (size 0.6) (drill 0.3) (layers "F.Cu" "B.Cu") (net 5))
 (segment (start 146.558 74.295) (end 146.558 75.518) (width 0.25) (layer "B.Cu") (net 5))
 (segment (start 138.049 75.5396) (end 138.049 74.295) (width 0.25) (layer "B.Cu") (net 5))
 (segment (start 146.558 68.2714) (end 146.558 69.596) (width 0.25) (layer "B.Cu") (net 5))
 (segment (start 141.4449 69.6214) (end 143.1439 69.6214) (width 0.25) (layer "B.Cu") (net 5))
 (segment (start 144.6784 58.8518) (end 149.5044 63.6778) (width 0.25) (layer "F.Cu") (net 8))
 (segment (start 144.2466 58.8518) (end 144.6784 58.8518) (width 0.25) (layer "F.Cu") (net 8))
 (via (at 149.5044 63.6778) (size 0.6) (drill 0.3) (layers "F.Cu" "B.Cu") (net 8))
 (segment (start 149.5044 66.4983) (end 149.5044 64.8716) (width 0.25) (layer "B.Cu") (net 8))
 (segment (start 149.5044 63.6778) (end 149.5044 64.8716) (width 0.25) (layer "B.Cu") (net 8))
 (segment (start 146.558 77.343) (end 144.8308 77.343) (width 0.25) (layer "B.Cu") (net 2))
 (segment (start 144.833 79.386) (end 144.833 77.3452) (width 0.25) (layer "B.Cu") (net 2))
 (segment (start 147.665 64.886) (end 146.5436 64.886) (width 0.25) (layer "B.Cu") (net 4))
 (segment (start 146.558 66.4464) (end 146.558 64.9004) (width 0.25) (layer "B.Cu") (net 4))
 (segment (start 146.5436 64.886) (end 144.833 64.886) (width 0.25) (layer "B.Cu") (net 4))
 (segment (start 146.558 64.9004) (end 146.5436 64.886) (width 0.25) (layer "B.Cu") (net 4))
 (segment (start 139.833 79.386) (end 139.833 77.3744) (width 0.25) (layer "B.Cu") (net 1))
 (segment (start 139.827 77.3684) (end 138.0528 77.3684) (width 0.25) (layer "B.Cu") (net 1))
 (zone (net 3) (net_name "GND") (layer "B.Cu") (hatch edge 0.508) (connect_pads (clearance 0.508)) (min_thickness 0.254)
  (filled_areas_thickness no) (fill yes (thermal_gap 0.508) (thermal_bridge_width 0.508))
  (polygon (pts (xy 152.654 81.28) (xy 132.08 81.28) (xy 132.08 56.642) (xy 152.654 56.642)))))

